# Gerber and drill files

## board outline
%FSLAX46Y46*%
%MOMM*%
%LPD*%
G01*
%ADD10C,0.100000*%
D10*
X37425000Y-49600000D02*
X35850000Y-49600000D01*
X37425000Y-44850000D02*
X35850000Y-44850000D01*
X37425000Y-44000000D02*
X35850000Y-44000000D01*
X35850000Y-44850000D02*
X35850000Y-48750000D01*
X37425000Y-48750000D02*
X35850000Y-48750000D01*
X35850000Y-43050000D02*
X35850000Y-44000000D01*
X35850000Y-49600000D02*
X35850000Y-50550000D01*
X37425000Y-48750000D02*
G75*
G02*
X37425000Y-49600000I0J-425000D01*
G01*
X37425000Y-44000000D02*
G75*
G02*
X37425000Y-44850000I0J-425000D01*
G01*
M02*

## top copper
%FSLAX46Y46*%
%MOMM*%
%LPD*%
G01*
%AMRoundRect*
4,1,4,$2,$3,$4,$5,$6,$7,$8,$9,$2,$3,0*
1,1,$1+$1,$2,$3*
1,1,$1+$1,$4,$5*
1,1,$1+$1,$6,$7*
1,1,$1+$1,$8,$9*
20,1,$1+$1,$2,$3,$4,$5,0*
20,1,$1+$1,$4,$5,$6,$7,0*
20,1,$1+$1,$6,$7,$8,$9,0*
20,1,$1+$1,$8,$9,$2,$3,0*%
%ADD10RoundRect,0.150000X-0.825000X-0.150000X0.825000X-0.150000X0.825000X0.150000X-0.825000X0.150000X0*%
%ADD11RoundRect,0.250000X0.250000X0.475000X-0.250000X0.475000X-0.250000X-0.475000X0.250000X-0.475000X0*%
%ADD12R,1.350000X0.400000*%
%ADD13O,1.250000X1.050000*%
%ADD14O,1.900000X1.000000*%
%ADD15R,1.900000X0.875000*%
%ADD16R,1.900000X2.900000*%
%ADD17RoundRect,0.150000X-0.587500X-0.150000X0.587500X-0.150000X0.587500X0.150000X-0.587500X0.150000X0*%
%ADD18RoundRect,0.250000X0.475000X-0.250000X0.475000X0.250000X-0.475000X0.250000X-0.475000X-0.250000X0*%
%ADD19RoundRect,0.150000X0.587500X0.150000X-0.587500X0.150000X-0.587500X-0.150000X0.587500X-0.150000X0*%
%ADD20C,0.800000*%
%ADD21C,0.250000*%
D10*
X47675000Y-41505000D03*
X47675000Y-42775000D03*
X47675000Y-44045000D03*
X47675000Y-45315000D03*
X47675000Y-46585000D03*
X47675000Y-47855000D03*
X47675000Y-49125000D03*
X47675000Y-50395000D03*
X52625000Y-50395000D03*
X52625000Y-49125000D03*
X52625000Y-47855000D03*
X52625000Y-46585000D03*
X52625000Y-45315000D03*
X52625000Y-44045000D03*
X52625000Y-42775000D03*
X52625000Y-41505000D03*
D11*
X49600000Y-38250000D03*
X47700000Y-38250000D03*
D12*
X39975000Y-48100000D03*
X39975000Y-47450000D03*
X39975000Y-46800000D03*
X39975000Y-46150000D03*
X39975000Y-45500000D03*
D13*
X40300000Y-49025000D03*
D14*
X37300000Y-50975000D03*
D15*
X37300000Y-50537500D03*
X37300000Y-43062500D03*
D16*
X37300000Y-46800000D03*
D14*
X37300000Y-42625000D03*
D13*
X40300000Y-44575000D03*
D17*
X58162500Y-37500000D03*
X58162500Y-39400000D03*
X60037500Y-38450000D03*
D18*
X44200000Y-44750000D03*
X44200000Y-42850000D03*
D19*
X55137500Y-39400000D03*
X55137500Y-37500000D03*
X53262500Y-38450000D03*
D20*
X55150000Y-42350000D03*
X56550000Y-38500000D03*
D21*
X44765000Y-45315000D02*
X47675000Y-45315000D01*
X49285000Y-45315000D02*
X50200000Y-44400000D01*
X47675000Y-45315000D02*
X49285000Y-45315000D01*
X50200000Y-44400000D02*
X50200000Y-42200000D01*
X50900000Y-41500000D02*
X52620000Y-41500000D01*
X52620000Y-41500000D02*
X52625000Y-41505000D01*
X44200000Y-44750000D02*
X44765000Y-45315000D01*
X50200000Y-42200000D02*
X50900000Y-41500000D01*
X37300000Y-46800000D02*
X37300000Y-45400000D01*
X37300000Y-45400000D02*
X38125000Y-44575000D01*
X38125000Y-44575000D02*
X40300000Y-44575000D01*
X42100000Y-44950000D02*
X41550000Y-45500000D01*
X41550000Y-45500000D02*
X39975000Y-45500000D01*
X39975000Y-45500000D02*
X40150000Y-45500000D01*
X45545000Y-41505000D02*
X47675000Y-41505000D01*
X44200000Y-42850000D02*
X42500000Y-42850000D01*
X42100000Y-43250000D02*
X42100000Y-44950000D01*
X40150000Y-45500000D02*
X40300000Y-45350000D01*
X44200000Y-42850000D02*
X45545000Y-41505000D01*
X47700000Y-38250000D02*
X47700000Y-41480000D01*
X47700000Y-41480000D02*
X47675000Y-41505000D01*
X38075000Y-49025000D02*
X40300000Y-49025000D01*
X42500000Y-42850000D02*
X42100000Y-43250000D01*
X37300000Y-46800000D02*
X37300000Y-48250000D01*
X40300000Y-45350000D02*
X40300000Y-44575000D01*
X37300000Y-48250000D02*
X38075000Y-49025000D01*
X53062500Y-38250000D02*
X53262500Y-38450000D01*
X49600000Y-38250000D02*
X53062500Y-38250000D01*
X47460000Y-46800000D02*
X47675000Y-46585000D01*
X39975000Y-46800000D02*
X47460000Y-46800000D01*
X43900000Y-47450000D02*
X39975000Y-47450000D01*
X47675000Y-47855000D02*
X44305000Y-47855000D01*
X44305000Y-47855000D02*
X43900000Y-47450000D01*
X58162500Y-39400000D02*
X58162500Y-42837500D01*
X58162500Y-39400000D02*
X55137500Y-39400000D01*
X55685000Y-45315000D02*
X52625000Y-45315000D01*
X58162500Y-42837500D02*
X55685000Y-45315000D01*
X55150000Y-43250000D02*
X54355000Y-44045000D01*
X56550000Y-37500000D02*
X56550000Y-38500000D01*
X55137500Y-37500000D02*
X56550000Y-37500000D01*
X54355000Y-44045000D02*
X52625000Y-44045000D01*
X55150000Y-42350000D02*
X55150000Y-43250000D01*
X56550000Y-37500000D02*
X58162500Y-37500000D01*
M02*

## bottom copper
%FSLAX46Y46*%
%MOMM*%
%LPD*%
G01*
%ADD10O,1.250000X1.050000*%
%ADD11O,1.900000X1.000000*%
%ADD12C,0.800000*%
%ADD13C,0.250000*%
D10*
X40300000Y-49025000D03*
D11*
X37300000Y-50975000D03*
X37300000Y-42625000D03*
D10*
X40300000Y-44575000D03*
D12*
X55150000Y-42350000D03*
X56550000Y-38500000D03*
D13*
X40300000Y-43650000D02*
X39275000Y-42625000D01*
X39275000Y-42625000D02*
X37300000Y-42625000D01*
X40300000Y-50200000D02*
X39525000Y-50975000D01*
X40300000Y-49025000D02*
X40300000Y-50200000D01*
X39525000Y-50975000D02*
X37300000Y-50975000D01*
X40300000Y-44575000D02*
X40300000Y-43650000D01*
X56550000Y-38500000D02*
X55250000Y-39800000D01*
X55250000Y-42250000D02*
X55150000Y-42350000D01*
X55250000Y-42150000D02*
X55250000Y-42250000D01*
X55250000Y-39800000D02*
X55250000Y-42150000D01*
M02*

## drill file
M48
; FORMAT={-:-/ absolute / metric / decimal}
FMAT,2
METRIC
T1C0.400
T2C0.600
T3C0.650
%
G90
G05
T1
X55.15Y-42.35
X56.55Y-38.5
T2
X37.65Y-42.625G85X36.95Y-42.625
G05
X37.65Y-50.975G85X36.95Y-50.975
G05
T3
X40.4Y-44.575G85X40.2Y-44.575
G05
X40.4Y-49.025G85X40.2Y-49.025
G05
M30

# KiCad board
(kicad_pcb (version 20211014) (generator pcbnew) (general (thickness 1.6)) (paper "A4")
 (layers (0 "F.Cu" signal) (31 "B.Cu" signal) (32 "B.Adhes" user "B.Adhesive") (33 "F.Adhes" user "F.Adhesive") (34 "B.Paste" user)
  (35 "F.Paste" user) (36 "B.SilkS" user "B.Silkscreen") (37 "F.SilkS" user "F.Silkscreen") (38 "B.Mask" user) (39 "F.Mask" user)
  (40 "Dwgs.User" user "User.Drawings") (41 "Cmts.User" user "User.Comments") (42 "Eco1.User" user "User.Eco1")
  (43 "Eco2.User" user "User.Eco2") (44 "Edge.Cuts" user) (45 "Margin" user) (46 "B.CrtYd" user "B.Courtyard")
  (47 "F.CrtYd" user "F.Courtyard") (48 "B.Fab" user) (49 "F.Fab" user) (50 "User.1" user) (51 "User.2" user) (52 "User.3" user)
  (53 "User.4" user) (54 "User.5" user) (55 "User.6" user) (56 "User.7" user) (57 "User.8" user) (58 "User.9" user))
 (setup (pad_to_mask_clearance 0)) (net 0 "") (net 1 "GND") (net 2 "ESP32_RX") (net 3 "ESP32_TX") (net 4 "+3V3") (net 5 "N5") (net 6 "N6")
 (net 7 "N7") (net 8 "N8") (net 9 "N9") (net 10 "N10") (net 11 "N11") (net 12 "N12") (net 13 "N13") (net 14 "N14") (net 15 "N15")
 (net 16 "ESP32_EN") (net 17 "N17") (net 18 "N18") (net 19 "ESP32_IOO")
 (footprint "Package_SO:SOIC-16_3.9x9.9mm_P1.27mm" (layer "F.Cu") (at 50.15 45.95)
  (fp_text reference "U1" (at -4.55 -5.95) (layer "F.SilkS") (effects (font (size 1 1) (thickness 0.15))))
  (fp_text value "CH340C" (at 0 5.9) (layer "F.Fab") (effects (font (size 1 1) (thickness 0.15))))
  (pad "1" smd roundrect locked (at -2.475 -4.445) (size 1.95 0.6) (layers "F.Cu" "F.Paste" "F.Mask") (roundrect_rratio 0.25) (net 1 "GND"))
  (pad "2" smd roundrect locked (at -2.475 -3.175) (size 1.95 0.6) (layers "F.Cu" "F.Paste" "F.Mask") (roundrect_rratio 0.25)
   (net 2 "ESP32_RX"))
  (pad "3" smd roundrect locked (at -2.475 -1.905) (size 1.95 0.6) (layers "F.Cu" "F.Paste" "F.Mask") (roundrect_rratio 0.25)
   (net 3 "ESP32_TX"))
  (pad "4" smd roundrect locked (at -2.475 -0.635) (size 1.95 0.6) (layers "F.Cu" "F.Paste" "F.Mask") (roundrect_rratio 0.25) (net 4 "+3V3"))
  (pad "5" smd roundrect locked (at -2.475 0.635) (size 1.95 0.6) (layers "F.Cu" "F.Paste" "F.Mask") (roundrect_rratio 0.25) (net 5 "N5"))
  (pad "6" smd roundrect locked (at -2.475 1.905) (size 1.95 0.6) (layers "F.Cu" "F.Paste" "F.Mask") (roundrect_rratio 0.25) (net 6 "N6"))
  (pad "7" smd roundrect locked (at -2.475 3.175) (size 1.95 0.6) (layers "F.Cu" "F.Paste" "F.Mask") (roundrect_rratio 0.25) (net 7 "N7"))
  (pad "8" smd roundrect locked (at -2.475 4.445) (size 1.95 0.6) (layers "F.Cu" "F.Paste" "F.Mask") (roundrect_rratio 0.25) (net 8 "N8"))
  (pad "9" smd roundrect locked (at 2.475 4.445) (size 1.95 0.6) (layers "F.Cu" "F.Paste" "F.Mask") (roundrect_rratio 0.25) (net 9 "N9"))
  (pad "10" smd roundrect locked (at 2.475 3.175) (size 1.95 0.6) (layers "F.Cu" "F.Paste" "F.Mask") (roundrect_rratio 0.25) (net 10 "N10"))
  (pad "11" smd roundrect locked (at 2.475 1.905) (size 1.95 0.6) (layers "F.Cu" "F.Paste" "F.Mask") (roundrect_rratio 0.25) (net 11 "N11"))
  (pad "12" smd roundrect locked (at 2.475 0.635) (size 1.95 0.6) (layers "F.Cu" "F.Paste" "F.Mask") (roundrect_rratio 0.25) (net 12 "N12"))
  (pad "13" smd roundrect locked (at 2.475 -0.635) (size 1.95 0.6) (layers "F.Cu" "F.Paste" "F.Mask") (roundrect_rratio 0.25) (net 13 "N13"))
  (pad "14" smd roundrect locked (at 2.475 -1.905) (size 1.95 0.6) (layers "F.Cu" "F.Paste" "F.Mask") (roundrect_rratio 0.25) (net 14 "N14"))
  (pad "15" smd roundrect locked (at 2.475 -3.175) (size 1.95 0.6) (layers "F.Cu" "F.Paste" "F.Mask") (roundrect_rratio 0.25) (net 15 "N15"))
  (pad "16" smd roundrect locked (at 2.475 -4.445) (size 1.95 0.6) (layers "F.Cu" "F.Paste" "F.Mask") (roundrect_rratio 0.25) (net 4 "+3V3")))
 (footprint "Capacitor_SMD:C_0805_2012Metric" (layer "F.Cu") (at 48.65 38.25 180)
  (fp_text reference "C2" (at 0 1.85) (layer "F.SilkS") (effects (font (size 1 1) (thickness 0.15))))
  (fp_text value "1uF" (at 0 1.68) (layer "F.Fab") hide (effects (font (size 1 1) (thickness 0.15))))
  (pad "1" smd roundrect locked (at -0.95 0 180) (size 1 1.45) (layers "F.Cu" "F.Paste" "F.Mask") (roundrect_rratio 0.25)
   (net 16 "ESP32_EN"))
  (pad "2" smd roundrect locked (at 0.95 0 180) (size 1 1.45) (layers "F.Cu" "F.Paste" "F.Mask") (roundrect_rratio 0.25) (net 1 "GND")))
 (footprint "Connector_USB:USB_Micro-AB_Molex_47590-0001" (layer "F.Cu") (at 37.3 46.8 -90)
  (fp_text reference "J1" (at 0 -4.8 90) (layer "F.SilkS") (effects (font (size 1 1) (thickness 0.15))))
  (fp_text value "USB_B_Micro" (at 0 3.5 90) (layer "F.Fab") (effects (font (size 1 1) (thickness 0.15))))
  (fp_line (start 2.8 -0.125) (end 2.8 1.45) (layer "Edge.Cuts") (width 0.1))
  (fp_line (start -1.95 -0.125) (end -1.95 1.45) (layer "Edge.Cuts") (width 0.1))
  (fp_line (start -2.8 -0.125) (end -2.8 1.45) (layer "Edge.Cuts") (width 0.1))
  (fp_line (start -1.95 1.45) (end 1.95 1.45) (layer "Edge.Cuts") (width 0.1))
  (fp_line (start 1.95 -0.125) (end 1.95 1.45) (layer "Edge.Cuts") (width 0.1))
  (fp_line (start -3.75 1.45) (end -2.8 1.45) (layer "Edge.Cuts") (width 0.1))
  (fp_line (start 2.8 1.45) (end 3.75 1.45) (layer "Edge.Cuts") (width 0.1))
  (fp_arc (start 1.95 -0.125) (mid 2.375 -0.55) (end 2.8 -0.125) (layer "Edge.Cuts") (width 0.1))
  (fp_arc (start -2.8 -0.125) (mid -2.375 -0.55) (end -1.95 -0.125) (layer "Edge.Cuts") (width 0.1))
  (pad "" smd rect locked (at 3.5 0 270) (size 0.3 0.85) (layers "F.Paste"))
  (pad "" smd rect locked (at -3.5 0 270) (size 0.3 0.85) (layers "F.Paste"))
  (pad "1" smd rect locked (at 1.3 -2.675 270) (size 0.4 1.35) (layers "F.Cu" "F.Paste" "F.Mask") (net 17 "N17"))
  (pad "2" smd rect locked (at 0.65 -2.675 270) (size 0.4 1.35) (layers "F.Cu" "F.Paste" "F.Mask") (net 6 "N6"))
  (pad "3" smd rect locked (at 0 -2.675 270) (size 0.4 1.35) (layers "F.Cu" "F.Paste" "F.Mask") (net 5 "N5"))
  (pad "4" smd rect locked (at -0.65 -2.675 270) (size 0.4 1.35) (layers "F.Cu" "F.Paste" "F.Mask") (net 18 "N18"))
  (pad "5" smd rect locked (at -1.3 -2.675 270) (size 0.4 1.35) (layers "F.Cu" "F.Paste" "F.Mask") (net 1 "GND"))
  (pad "6" thru_hole oval locked (at 2.225 -3 270) (size 1.05 1.25) (drill oval 0.65 0.85) (layers *.Cu *.Mask) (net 1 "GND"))
  (pad "6" thru_hole oval locked (at 4.175 0 270) (size 1 1.9) (drill oval 0.6 1.3) (layers *.Cu *.Mask) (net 1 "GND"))
  (pad "6" smd rect locked (at 3.7375 0 270) (size 0.875 1.9) (layers "F.Cu" "F.Mask") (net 1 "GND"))
  (pad "6" smd rect locked (at -3.7375 0 270) (size 0.875 1.9) (layers "F.Cu" "F.Mask") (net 1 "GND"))
  (pad "6" smd rect locked (at 0 0 270) (size 2.9 1.9) (layers "F.Cu" "F.Paste" "F.Mask") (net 1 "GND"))
  (pad "6" thru_hole oval locked (at -4.175 0 270) (size 1 1.9) (drill oval 0.6 1.3) (layers *.Cu *.Mask) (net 1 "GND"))
  (pad "6" thru_hole oval locked (at -2.225 -3 270) (size 1.05 1.25) (drill oval 0.65 0.85) (layers *.Cu *.Mask) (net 1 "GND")))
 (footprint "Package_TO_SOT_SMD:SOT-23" (layer "F.Cu") (at 59.1 38.45)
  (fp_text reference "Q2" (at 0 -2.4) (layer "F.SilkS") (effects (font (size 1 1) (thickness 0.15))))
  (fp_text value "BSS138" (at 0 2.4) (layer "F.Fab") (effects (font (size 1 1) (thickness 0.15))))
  (pad "1" smd roundrect locked (at -0.9375 -0.95) (size 1.475 0.6) (layers "F.Cu" "F.Paste" "F.Mask") (roundrect_rratio 0.25)
   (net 14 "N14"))
  (pad "2" smd roundrect locked (at -0.9375 0.95) (size 1.475 0.6) (layers "F.Cu" "F.Paste" "F.Mask") (roundrect_rratio 0.25) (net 13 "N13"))
  (pad "3" smd roundrect locked (at 0.9375 0) (size 1.475 0.6) (layers "F.Cu" "F.Paste" "F.Mask") (roundrect_rratio 0.25)
   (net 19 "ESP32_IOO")))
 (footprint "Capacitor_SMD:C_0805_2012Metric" (layer "F.Cu") (at 44.2 43.8 90)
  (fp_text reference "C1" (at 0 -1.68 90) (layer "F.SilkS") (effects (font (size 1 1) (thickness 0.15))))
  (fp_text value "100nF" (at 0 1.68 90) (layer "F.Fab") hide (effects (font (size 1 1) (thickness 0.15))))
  (pad "1" smd roundrect locked (at -0.95 0 90) (size 1 1.45) (layers "F.Cu" "F.Paste" "F.Mask") (roundrect_rratio 0.25) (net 4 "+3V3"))
  (pad "2" smd roundrect locked (at 0.95 0 90) (size 1 1.45) (layers "F.Cu" "F.Paste" "F.Mask") (roundrect_rratio 0.25) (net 1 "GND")))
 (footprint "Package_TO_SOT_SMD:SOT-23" (layer "F.Cu") (at 54.2 38.45 180)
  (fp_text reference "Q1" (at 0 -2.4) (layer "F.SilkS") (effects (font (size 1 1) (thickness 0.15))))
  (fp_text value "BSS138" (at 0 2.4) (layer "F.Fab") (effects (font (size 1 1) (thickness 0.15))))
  (pad "1" smd roundrect locked (at -0.9375 -0.95 180) (size 1.475 0.6) (layers "F.Cu" "F.Paste" "F.Mask") (roundrect_rratio 0.25)
   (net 13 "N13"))
  (pad "2" smd roundrect locked (at -0.9375 0.95 180) (size 1.475 0.6) (layers "F.Cu" "F.Paste" "F.Mask") (roundrect_rratio 0.25)
   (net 14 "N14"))
  (pad "3" smd roundrect locked (at 0.9375 0 180) (size 1.475 0.6) (layers "F.Cu" "F.Paste" "F.Mask") (roundrect_rratio 0.25)
   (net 16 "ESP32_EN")))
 (segment (start 44.765 45.315) (end 47.675 45.315) (width 0.25) (layer "F.Cu") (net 4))
 (segment (start 49.285 45.315) (end 50.2 44.4) (width 0.25) (layer "F.Cu") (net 4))
 (segment (start 47.675 45.315) (end 49.285 45.315) (width 0.25) (layer "F.Cu") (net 4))
 (segment (start 50.2 44.4) (end 50.2 42.2) (width 0.25) (layer "F.Cu") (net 4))
 (segment (start 50.9 41.5) (end 52.62 41.5) (width 0.25) (layer "F.Cu") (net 4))
 (segment (start 52.62 41.5) (end 52.625 41.505) (width 0.25) (layer "F.Cu") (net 4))
 (segment (start 44.2 44.75) (end 44.765 45.315) (width 0.25) (layer "F.Cu") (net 4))
 (segment (start 50.2 42.2) (end 50.9 41.5) (width 0.25) (layer "F.Cu") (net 4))
 (segment (start 37.3 46.8) (end 37.3 45.4) (width 0.25) (layer "F.Cu") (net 1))
 (segment (start 37.3 45.4) (end 38.125 44.575) (width 0.25) (layer "F.Cu") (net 1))
 (segment (start 38.125 44.575) (end 40.3 44.575) (width 0.25) (layer "F.Cu") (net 1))
 (segment (start 42.1 44.95) (end 41.55 45.5) (width 0.25) (layer "F.Cu") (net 1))
 (segment (start 41.55 45.5) (end 39.975 45.5) (width 0.25) (layer "F.Cu") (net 1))
 (segment (start 39.975 45.5) (end 40.15 45.5) (width 0.25) (layer "F.Cu") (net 1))
 (segment (start 45.545 41.505) (end 47.675 41.505) (width 0.25) (layer "F.Cu") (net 1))
 (segment (start 44.2 42.85) (end 42.5 42.85) (width 0.25) (layer "F.Cu") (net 1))
 (segment (start 42.1 43.25) (end 42.1 44.95) (width 0.25) (layer "F.Cu") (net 1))
 (segment (start 40.15 45.5) (end 40.3 45.35) (width 0.25) (layer "F.Cu") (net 1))
 (segment (start 44.2 42.85) (end 45.545 41.505) (width 0.25) (layer "F.Cu") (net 1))
 (segment (start 47.7 38.25) (end 47.7 41.48) (width 0.25) (layer "F.Cu") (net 1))
 (segment (start 47.7 41.48) (end 47.675 41.505) (width 0.25) (layer "F.Cu") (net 1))
 (segment (start 38.075 49.025) (end 40.3 49.025) (width 0.25) (layer "F.Cu") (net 1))
 (segment (start 42.5 42.85) (end 42.1 43.25) (width 0.25) (layer "F.Cu") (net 1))
 (segment (start 37.3 46.8) (end 37.3 48.25) (width 0.25) (layer "F.Cu") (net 1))
 (segment (start 40.3 45.35) (end 40.3 44.575) (width 0.25) (layer "F.Cu") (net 1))
 (segment (start 37.3 48.25) (end 38.075 49.025) (width 0.25) (layer "F.Cu") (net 1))
 (segment (start 40.3 43.65) (end 39.275 42.625) (width 0.25) (layer "B.Cu") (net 1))
 (segment (start 39.275 42.625) (end 37.3 42.625) (width 0.25) (layer "B.Cu") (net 1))
 (segment (start 40.3 50.2) (end 39.525 50.975) (width 0.25) (layer "B.Cu") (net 1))
 (segment (start 40.3 49.025) (end 40.3 50.2) (width 0.25) (layer "B.Cu") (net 1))
 (segment (start 39.525 50.975) (end 37.3 50.975) (width 0.25) (layer "B.Cu") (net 1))
 (segment (start 40.3 44.575) (end 40.3 43.65) (width 0.25) (layer "B.Cu") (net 1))
 (segment (start 53.0625 38.25) (end 53.2625 38.45) (width 0.25) (layer "F.Cu") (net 16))
 (segment (start 49.6 38.25) (end 53.0625 38.25) (width 0.25) (layer "F.Cu") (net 16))
 (segment (start 47.46 46.8) (end 47.675 46.585) (width 0.25) (layer "F.Cu") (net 5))
 (segment (start 39.975 46.8) (end 47.46 46.8) (width 0.25) (layer "F.Cu") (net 5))
 (segment (start 43.9 47.45) (end 39.975 47.45) (width 0.25) (layer "F.Cu") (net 6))
 (segment (start 47.675 47.855) (end 44.305 47.855) (width 0.25) (layer "F.Cu") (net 6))
 (segment (start 44.305 47.855) (end 43.9 47.45) (width 0.25) (layer "F.Cu") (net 6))
 (segment (start 58.1625 39.4) (end 58.1625 42.8375) (width 0.25) (layer "F.Cu") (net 13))
 (segment (start 58.1625 39.4) (end 55.1375 39.4) (width 0.25) (layer "F.Cu") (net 13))
 (segment (start 55.685 45.315) (end 52.625 45.315) (width 0.25) (layer "F.Cu") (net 13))
 (segment (start 58.1625 42.8375) (end 55.685 45.315) (width 0.25) (layer "F.Cu") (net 13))
 (segment (start 55.15 43.25) (end 54.355 44.045) (width 0.25) (layer "F.Cu") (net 14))
 (segment (start 56.55 37.5) (end 56.55 38.5) (width 0.25) (layer "F.Cu") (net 14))
 (segment (start 55.1375 37.5) (end 56.55 37.5) (width 0.25) (layer "F.Cu") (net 14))
 (segment (start 54.355 44.045) (end 52.625 44.045) (width 0.25) (layer "F.Cu") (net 14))
 (segment (start 55.15 42.35) (end 55.15 43.25) (width 0.25) (layer "F.Cu") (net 14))
 (segment (start 56.55 37.5) (end 58.1625 37.5) (width 0.25) (layer "F.Cu") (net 14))
 (via (at 55.15 42.35) (size 0.8) (drill 0.4) (layers "F.Cu" "B.Cu") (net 14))
 (via (at 56.55 38.5) (size 0.8) (drill 0.4) (layers "F.Cu" "B.Cu") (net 14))
 (segment (start 56.55 38.5) (end 55.25 39.8) (width 0.25) (layer "B.Cu") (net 14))
 (segment (start 55.25 42.25) (end 55.15 42.35) (width 0.25) (layer "B.Cu") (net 14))
 (segment (start 55.25 42.15) (end 55.25 42.25) (width 0.25) (layer "B.Cu") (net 14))
 (segment (start 55.25 39.8) (end 55.25 42.15) (width 0.25) (layer "B.Cu") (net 14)))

